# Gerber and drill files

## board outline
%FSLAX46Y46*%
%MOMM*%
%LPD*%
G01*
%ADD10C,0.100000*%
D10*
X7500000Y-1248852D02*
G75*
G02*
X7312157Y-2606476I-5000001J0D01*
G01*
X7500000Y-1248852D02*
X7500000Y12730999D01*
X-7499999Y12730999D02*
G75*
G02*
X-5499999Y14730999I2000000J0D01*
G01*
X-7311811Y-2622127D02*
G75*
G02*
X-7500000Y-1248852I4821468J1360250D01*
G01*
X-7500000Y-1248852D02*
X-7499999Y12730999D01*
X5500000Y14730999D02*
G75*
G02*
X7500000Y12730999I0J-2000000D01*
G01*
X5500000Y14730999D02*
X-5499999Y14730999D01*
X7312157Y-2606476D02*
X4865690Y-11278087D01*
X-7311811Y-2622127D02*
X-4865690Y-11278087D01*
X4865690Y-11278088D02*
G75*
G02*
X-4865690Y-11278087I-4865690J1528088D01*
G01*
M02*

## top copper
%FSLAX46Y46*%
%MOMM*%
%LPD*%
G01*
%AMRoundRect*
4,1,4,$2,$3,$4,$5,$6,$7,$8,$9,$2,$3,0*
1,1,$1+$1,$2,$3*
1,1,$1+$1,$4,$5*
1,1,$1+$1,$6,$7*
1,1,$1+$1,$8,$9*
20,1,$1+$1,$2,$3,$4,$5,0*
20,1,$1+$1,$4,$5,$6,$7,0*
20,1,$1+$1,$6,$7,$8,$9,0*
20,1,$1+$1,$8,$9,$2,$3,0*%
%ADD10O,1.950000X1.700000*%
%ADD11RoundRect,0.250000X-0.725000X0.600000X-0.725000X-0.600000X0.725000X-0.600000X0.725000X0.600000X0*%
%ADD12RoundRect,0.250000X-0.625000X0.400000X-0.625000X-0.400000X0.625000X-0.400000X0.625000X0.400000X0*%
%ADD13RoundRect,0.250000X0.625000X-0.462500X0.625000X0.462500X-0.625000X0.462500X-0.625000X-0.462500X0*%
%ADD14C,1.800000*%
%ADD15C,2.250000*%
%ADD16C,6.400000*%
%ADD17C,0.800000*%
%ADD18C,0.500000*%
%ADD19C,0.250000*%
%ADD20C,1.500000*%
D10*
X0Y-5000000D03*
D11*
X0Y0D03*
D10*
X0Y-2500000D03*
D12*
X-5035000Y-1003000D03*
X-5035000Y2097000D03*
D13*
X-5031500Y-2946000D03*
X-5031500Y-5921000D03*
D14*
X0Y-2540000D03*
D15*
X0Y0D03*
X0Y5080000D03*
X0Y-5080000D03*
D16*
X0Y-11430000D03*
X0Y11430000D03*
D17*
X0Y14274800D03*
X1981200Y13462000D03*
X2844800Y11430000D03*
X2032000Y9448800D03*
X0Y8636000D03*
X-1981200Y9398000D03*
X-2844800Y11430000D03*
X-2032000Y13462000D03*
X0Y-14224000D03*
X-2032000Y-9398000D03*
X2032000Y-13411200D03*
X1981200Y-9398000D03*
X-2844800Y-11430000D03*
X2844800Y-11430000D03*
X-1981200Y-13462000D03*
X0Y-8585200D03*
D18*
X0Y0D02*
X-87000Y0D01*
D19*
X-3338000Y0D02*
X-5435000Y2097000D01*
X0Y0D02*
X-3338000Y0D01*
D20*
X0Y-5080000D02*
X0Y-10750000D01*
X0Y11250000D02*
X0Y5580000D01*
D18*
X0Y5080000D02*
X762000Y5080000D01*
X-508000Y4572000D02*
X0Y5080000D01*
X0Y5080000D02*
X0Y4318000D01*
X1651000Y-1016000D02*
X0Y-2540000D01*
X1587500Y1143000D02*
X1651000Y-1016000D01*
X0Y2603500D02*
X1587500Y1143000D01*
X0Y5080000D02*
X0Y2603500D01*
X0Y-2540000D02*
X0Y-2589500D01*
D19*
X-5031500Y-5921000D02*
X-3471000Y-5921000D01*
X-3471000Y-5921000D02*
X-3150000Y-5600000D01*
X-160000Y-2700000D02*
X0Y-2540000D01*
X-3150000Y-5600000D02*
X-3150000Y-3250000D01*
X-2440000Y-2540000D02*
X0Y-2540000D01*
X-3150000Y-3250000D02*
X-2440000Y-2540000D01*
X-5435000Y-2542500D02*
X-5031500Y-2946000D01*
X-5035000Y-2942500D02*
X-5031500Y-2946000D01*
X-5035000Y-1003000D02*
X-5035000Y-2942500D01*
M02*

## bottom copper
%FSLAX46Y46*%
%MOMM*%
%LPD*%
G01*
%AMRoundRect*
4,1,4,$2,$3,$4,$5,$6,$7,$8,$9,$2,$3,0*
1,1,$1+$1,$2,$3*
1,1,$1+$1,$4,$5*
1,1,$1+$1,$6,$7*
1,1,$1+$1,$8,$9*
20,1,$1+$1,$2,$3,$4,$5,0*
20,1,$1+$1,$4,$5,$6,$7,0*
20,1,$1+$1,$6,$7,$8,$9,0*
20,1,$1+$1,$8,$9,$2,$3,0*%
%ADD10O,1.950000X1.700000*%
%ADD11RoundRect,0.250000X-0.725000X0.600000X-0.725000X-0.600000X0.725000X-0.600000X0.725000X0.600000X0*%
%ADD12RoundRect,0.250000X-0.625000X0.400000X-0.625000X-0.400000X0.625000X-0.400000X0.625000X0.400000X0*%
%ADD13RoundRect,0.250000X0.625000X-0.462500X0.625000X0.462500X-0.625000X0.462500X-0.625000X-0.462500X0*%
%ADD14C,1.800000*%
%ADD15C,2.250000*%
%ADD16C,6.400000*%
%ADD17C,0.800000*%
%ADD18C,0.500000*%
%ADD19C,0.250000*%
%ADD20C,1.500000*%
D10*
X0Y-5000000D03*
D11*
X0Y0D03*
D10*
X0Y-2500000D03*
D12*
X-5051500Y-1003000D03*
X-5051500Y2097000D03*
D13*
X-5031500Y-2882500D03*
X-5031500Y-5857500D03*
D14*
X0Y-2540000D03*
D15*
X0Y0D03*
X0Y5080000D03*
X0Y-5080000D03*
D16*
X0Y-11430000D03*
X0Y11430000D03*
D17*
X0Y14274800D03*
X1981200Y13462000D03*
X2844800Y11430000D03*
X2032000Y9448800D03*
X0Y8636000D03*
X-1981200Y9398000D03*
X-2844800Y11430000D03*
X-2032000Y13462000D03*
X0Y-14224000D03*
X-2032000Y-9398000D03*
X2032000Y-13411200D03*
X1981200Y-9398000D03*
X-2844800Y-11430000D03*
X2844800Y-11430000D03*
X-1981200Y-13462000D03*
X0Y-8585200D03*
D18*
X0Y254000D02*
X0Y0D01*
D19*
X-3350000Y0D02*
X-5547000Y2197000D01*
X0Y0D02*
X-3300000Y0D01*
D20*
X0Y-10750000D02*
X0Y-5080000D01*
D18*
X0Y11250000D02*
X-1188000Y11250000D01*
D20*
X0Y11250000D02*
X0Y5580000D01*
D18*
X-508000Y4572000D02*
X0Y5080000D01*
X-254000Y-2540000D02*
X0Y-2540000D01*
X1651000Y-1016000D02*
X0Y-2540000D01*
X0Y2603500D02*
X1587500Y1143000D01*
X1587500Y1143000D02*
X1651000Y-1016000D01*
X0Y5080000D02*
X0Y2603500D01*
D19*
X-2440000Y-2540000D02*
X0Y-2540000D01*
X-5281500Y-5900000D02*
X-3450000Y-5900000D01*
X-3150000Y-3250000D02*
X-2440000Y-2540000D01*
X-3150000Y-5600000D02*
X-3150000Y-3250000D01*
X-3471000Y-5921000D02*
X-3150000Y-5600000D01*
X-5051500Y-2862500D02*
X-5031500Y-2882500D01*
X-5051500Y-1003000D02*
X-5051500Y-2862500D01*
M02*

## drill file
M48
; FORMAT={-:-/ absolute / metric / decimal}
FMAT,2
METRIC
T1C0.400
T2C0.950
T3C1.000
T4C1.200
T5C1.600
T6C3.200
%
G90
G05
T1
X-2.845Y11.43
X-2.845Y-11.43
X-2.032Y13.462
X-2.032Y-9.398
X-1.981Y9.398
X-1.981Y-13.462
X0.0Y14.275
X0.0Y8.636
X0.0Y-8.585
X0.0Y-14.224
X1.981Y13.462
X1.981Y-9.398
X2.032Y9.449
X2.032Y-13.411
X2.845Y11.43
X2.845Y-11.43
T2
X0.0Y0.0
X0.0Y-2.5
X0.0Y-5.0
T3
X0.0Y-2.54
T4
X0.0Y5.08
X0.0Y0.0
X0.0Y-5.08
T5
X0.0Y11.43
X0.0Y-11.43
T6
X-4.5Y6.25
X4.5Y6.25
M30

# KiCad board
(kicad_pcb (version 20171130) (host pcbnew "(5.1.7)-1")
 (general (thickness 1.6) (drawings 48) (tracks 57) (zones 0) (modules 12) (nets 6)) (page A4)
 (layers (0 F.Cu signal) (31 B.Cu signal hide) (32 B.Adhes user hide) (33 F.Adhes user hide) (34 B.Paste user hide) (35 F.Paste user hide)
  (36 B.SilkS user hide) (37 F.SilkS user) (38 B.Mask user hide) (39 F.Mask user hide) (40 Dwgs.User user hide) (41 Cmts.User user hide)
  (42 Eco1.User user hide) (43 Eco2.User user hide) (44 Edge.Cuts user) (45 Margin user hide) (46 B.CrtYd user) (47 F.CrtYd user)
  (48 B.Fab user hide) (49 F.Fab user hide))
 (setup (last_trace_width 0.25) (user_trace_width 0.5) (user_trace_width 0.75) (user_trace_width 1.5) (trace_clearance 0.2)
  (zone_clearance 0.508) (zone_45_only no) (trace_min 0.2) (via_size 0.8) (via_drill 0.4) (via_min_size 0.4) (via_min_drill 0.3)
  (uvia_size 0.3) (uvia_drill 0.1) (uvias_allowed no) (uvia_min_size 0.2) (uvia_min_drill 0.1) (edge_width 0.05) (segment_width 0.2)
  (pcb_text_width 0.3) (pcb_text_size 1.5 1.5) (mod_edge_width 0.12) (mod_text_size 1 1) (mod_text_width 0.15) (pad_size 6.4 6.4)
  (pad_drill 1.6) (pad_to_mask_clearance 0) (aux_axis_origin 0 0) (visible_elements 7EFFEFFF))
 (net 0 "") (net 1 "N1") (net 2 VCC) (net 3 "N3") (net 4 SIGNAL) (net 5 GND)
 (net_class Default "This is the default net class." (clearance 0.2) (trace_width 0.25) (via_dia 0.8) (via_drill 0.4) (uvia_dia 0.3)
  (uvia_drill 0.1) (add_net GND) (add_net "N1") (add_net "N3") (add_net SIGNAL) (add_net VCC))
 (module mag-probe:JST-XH (layer F.Cu) (at 0 0 270)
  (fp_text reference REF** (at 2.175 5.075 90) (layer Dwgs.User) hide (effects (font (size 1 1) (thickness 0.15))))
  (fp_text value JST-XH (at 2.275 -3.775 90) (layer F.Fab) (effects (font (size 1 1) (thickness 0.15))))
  (pad 3 thru_hole oval (at 5 0 270) (size 1.7 1.95) (drill 0.95) (layers *.Cu *.Mask))
  (pad 1 thru_hole roundrect (at 0 0 270) (size 1.7 1.95) (drill 0.95) (layers *.Cu *.Mask) (roundrect_rratio 0.147059))
  (pad 2 thru_hole oval (at 2.5 0 270) (size 1.7 1.95) (drill 0.95) (layers *.Cu *.Mask)))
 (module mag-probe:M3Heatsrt (layer F.Cu) (at -4.45 -6.3)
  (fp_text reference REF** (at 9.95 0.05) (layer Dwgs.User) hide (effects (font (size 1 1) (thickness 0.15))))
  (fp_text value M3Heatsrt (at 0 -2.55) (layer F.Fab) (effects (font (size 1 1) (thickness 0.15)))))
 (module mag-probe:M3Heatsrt (layer F.Cu) (at 4.45 -6.35)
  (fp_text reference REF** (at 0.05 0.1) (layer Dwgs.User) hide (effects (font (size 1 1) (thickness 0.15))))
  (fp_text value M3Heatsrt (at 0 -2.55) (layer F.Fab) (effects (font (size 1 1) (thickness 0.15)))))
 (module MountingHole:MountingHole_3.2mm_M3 (layer F.Cu) (at -4.6 -6.25)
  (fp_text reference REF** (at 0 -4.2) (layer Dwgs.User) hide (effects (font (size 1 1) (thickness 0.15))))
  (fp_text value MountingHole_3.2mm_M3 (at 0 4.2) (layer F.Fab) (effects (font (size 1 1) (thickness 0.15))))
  (pad "" np_thru_hole circle (at 0.1 0) (size 3.2 3.2) (drill 3.2) (layers *.Cu *.Mask)))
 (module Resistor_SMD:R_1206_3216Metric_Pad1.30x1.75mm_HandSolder (layer F.Cu) (at -5.035 -0.547 270)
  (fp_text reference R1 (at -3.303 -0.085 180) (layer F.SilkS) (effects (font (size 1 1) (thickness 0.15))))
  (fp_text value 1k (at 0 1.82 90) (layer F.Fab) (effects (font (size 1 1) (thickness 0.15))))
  (pad 2 smd roundrect (at 1.55 0 270) (size 1.3 1.75) (layers F.Cu F.Paste F.Mask) (roundrect_rratio 0.1923076923076923) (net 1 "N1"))
  (pad 1 smd roundrect (at -1.55 0 270) (size 1.3 1.75) (layers F.Cu F.Paste F.Mask) (roundrect_rratio 0.1923076923076923) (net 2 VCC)))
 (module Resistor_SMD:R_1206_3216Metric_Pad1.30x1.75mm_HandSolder (layer B.Cu) (at -5.0515 -0.547 270)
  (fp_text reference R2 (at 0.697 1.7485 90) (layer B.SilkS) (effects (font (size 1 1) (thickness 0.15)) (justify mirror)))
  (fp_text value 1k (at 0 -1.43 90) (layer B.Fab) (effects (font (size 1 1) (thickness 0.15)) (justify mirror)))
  (pad 2 smd roundrect (at 1.55 0 270) (size 1.3 1.75) (layers B.Cu B.Paste B.Mask) (roundrect_rratio 0.1923076923076923) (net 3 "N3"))
  (pad 1 smd roundrect (at -1.55 0 270) (size 1.3 1.75) (layers B.Cu B.Paste B.Mask) (roundrect_rratio 0.1923076923076923) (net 2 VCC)))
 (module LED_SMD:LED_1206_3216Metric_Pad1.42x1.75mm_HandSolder (layer F.Cu) (at -5.0315 4.4335 90)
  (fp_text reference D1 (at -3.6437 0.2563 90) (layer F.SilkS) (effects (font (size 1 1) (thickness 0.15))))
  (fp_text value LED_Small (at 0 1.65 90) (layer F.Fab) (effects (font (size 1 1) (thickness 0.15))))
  (pad 2 smd roundrect (at 1.4875 0 90) (size 1.425 1.75) (layers F.Cu F.Paste F.Mask) (roundrect_rratio 0.1754385964912281) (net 1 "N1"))
  (pad 1 smd roundrect (at -1.4875 0 90) (size 1.425 1.75) (layers F.Cu F.Paste F.Mask) (roundrect_rratio 0.1754385964912281) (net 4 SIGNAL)))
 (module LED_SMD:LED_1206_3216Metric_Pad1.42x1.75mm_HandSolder (layer B.Cu) (at -5.0315 4.37 90)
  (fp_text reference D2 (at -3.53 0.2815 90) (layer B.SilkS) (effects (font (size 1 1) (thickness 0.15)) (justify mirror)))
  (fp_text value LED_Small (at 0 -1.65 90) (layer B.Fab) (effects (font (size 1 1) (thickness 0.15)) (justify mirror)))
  (pad 2 smd roundrect (at 1.4875 0 90) (size 1.425 1.75) (layers B.Cu B.Paste B.Mask) (roundrect_rratio 0.1754385964912281) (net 3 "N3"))
  (pad 1 smd roundrect (at -1.4875 0 90) (size 1.425 1.75) (layers B.Cu B.Paste B.Mask) (roundrect_rratio 0.1754385964912281) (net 4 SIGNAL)))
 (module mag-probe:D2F (layer F.Cu) (at 0 0 270)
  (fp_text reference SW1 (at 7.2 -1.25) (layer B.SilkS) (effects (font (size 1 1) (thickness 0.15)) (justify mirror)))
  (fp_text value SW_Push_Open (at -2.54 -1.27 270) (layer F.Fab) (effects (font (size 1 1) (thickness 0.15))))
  (pad 4 thru_hole circle (at 2.54 0 270) (size 1.8 1.8) (drill 1) (layers *.Cu *.Mask) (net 4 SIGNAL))
  (pad 3 thru_hole circle (at 0 0 270) (size 2.25 2.25) (drill 1.2) (layers *.Cu *.Mask) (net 2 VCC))
  (pad 2 thru_hole circle (at -5.08 0 270) (size 2.25 2.25) (drill 1.2) (layers *.Cu *.Mask) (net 4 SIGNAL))
  (pad 1 thru_hole circle (at 5.08 0 270) (size 2.25 2.25) (drill 1.2) (layers *.Cu *.Mask) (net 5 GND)))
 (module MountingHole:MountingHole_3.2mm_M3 (layer F.Cu) (at 4.5 -6.25)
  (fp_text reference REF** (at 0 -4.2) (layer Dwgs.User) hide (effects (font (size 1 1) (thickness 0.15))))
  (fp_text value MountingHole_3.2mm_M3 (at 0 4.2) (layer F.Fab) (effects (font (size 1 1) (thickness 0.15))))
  (pad 1 np_thru_hole circle (at 0 0) (size 3.2 3.2) (drill 3.2) (layers *.Cu *.Mask)))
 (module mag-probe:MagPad (layer F.Cu) (at 0 11.25)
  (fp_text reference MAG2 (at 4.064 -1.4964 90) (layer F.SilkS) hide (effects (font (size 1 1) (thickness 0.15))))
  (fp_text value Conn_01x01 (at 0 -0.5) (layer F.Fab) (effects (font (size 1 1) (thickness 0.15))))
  (pad 1 thru_hole circle (at 0 0.18) (size 6.4 6.4) (drill 1.6) (layers *.Cu *.Mask) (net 5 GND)))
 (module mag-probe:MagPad (layer F.Cu) (at 0 -11.25)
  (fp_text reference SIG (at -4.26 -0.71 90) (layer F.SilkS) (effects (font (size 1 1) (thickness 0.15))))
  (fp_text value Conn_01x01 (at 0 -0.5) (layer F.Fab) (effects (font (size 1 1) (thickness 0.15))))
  (pad 1 thru_hole circle (at 0 -0.18) (size 6.4 6.4) (drill 1.6) (layers *.Cu *.Mask) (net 4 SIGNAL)))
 (gr_arc (start 2.499999 1.248852) (end 7.312157 2.606476) (angle -15.75501346) (layer Edge.Cuts) (width 0.1))
 (gr_line (start 7.5 1.248852) (end 7.5 -12.730999) (layer Edge.Cuts) (width 0.1))
 (gr_arc (start -5.499999 -12.730999) (end -5.499999 -14.730999) (angle -90) (layer Edge.Cuts) (width 0.1))
 (gr_arc (start -2.490343 1.261877) (end -7.5 1.248852) (angle -15.90398022) (layer Edge.Cuts) (width 0.1))
 (gr_line (start -7.5 1.248852) (end -7.499999 -12.730999) (layer Edge.Cuts) (width 0.1))
 (gr_arc (start 5.5 -12.730999) (end 7.5 -12.730999) (angle -90) (layer Edge.Cuts) (width 0.1))
 (gr_line (start 5.5 -14.730999) (end -5.499999 -14.730999) (layer Edge.Cuts) (width 0.1))
 (gr_line (start 7.312157 2.606476) (end 4.86569 11.278087) (layer Edge.Cuts) (width 0.1))
 (gr_line (start -7.311811 2.622127) (end -4.86569 11.278087) (layer Edge.Cuts) (width 0.1))
 (gr_arc (start 0 9.75) (end -4.86569 11.278087) (angle -145.1298326) (layer Edge.Cuts) (width 0.1))
 (via (at 0 -14.2748) (size 0.8) (drill 0.4) (layers F.Cu B.Cu) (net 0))
 (via (at 1.9812 -13.462) (size 0.8) (drill 0.4) (layers F.Cu B.Cu) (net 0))
 (via (at 2.8448 -11.43) (size 0.8) (drill 0.4) (layers F.Cu B.Cu) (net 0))
 (via (at 2.032 -9.4488) (size 0.8) (drill 0.4) (layers F.Cu B.Cu) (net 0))
 (via (at 0 -8.636) (size 0.8) (drill 0.4) (layers F.Cu B.Cu) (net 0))
 (via (at -1.9812 -9.398) (size 0.8) (drill 0.4) (layers F.Cu B.Cu) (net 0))
 (via (at -2.8448 -11.43) (size 0.8) (drill 0.4) (layers F.Cu B.Cu) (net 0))
 (via (at -2.032 -13.462) (size 0.8) (drill 0.4) (layers F.Cu B.Cu) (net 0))
 (via (at 0 14.224) (size 0.8) (drill 0.4) (layers F.Cu B.Cu) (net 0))
 (via (at -2.032 9.398) (size 0.8) (drill 0.4) (layers F.Cu B.Cu) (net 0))
 (via (at 2.032 13.4112) (size 0.8) (drill 0.4) (layers F.Cu B.Cu) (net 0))
 (via (at 1.9812 9.398) (size 0.8) (drill 0.4) (layers F.Cu B.Cu) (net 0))
 (via (at -2.8448 11.43) (size 0.8) (drill 0.4) (layers F.Cu B.Cu) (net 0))
 (via (at 2.8448 11.43) (size 0.8) (drill 0.4) (layers F.Cu B.Cu) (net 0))
 (via (at -1.9812 13.462) (size 0.8) (drill 0.4) (layers F.Cu B.Cu) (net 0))
 (via (at 0 8.5852) (size 0.8) (drill 0.4) (layers F.Cu B.Cu) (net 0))
 (segment (start 0 -0.254) (end 0 0) (width 0.5) (layer B.Cu) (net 2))
 (segment (start 0 0) (end -0.087 0) (width 0.5) (layer F.Cu) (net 2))
 (segment (start -3.338 0) (end -5.435 -2.097) (width 0.25) (layer F.Cu) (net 2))
 (segment (start 0 0) (end -3.338 0) (width 0.25) (layer F.Cu) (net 2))
 (segment (start -3.35 0) (end -5.547 -2.197) (width 0.25) (layer B.Cu) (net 2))
 (segment (start 0 0) (end -3.3 0) (width 0.25) (layer B.Cu) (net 2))
 (segment (start 0 10.75) (end 0 5.08) (width 1.5) (layer B.Cu) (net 5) (status 30))
 (segment (start 0 5.08) (end 0 10.75) (width 1.5) (layer F.Cu) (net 5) (status 30))
 (segment (start 0 -11.25) (end -1.188 -11.25) (width 0.5) (layer B.Cu) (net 4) (status 30))
 (segment (start 0 -11.25) (end 0 -5.58) (width 1.5) (layer B.Cu) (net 4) (status 30))
 (segment (start -0.508 -4.572) (end 0 -5.08) (width 0.5) (layer B.Cu) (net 4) (status 30))
 (segment (start 0 -11.25) (end 0 -5.58) (width 1.5) (layer F.Cu) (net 4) (status 30))
 (segment (start 0 -5.08) (end 0.762 -5.08) (width 0.5) (layer F.Cu) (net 4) (status 30))
 (segment (start -0.508 -4.572) (end 0 -5.08) (width 0.5) (layer F.Cu) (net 4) (status 30))
 (segment (start -0.254 2.54) (end 0 2.54) (width 0.5) (layer B.Cu) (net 4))
 (segment (start 0 -5.08) (end 0 -4.318) (width 0.5) (layer F.Cu) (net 4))
 (segment (start 1.651 1.016) (end 0 2.54) (width 0.5) (layer F.Cu) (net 4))
 (segment (start 1.5875 -1.143) (end 1.651 1.016) (width 0.5) (layer F.Cu) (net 4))
 (segment (start 0 -2.6035) (end 1.5875 -1.143) (width 0.5) (layer F.Cu) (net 4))
 (segment (start 1.651 1.016) (end 0 2.54) (width 0.5) (layer B.Cu) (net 4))
 (segment (start 0 -2.6035) (end 1.5875 -1.143) (width 0.5) (layer B.Cu) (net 4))
 (segment (start 1.5875 -1.143) (end 1.651 1.016) (width 0.5) (layer B.Cu) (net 4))
 (segment (start 0 -5.08) (end 0 -2.6035) (width 0.5) (layer B.Cu) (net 4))
 (segment (start 0 -5.08) (end 0 -2.6035) (width 0.5) (layer F.Cu) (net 4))
 (segment (start 0 2.54) (end 0 2.5895) (width 0.5) (layer F.Cu) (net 4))
 (segment (start -5.0315 5.921) (end -3.471 5.921) (width 0.25) (layer F.Cu) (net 4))
 (segment (start -3.471 5.921) (end -3.15 5.6) (width 0.25) (layer F.Cu) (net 4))
 (segment (start -0.16 2.7) (end 0 2.54) (width 0.25) (layer F.Cu) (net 4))
 (segment (start -3.15 5.6) (end -3.15 3.25) (width 0.25) (layer F.Cu) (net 4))
 (segment (start -2.44 2.54) (end 0 2.54) (width 0.25) (layer F.Cu) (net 4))
 (segment (start -3.15 3.25) (end -2.44 2.54) (width 0.25) (layer F.Cu) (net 4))
 (segment (start -2.44 2.54) (end 0 2.54) (width 0.25) (layer B.Cu) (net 4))
 (segment (start -5.2815 5.9) (end -3.45 5.9) (width 0.25) (layer B.Cu) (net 4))
 (segment (start -3.15 3.25) (end -2.44 2.54) (width 0.25) (layer B.Cu) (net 4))
 (segment (start -3.15 5.6) (end -3.15 3.25) (width 0.25) (layer B.Cu) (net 4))
 (segment (start -3.471 5.921) (end -3.15 5.6) (width 0.25) (layer B.Cu) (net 4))
 (segment (start -5.435 2.5425) (end -5.0315 2.946) (width 0.25) (layer F.Cu) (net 1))
 (segment (start -5.035 2.9425) (end -5.0315 2.946) (width 0.25) (layer F.Cu) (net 1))
 (segment (start -5.035 1.003) (end -5.035 2.9425) (width 0.25) (layer F.Cu) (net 1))
 (segment (start -5.0515 2.8625) (end -5.0315 2.8825) (width 0.25) (layer B.Cu) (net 3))
 (segment (start -5.0515 1.003) (end -5.0515 2.8625) (width 0.25) (layer B.Cu) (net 3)))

